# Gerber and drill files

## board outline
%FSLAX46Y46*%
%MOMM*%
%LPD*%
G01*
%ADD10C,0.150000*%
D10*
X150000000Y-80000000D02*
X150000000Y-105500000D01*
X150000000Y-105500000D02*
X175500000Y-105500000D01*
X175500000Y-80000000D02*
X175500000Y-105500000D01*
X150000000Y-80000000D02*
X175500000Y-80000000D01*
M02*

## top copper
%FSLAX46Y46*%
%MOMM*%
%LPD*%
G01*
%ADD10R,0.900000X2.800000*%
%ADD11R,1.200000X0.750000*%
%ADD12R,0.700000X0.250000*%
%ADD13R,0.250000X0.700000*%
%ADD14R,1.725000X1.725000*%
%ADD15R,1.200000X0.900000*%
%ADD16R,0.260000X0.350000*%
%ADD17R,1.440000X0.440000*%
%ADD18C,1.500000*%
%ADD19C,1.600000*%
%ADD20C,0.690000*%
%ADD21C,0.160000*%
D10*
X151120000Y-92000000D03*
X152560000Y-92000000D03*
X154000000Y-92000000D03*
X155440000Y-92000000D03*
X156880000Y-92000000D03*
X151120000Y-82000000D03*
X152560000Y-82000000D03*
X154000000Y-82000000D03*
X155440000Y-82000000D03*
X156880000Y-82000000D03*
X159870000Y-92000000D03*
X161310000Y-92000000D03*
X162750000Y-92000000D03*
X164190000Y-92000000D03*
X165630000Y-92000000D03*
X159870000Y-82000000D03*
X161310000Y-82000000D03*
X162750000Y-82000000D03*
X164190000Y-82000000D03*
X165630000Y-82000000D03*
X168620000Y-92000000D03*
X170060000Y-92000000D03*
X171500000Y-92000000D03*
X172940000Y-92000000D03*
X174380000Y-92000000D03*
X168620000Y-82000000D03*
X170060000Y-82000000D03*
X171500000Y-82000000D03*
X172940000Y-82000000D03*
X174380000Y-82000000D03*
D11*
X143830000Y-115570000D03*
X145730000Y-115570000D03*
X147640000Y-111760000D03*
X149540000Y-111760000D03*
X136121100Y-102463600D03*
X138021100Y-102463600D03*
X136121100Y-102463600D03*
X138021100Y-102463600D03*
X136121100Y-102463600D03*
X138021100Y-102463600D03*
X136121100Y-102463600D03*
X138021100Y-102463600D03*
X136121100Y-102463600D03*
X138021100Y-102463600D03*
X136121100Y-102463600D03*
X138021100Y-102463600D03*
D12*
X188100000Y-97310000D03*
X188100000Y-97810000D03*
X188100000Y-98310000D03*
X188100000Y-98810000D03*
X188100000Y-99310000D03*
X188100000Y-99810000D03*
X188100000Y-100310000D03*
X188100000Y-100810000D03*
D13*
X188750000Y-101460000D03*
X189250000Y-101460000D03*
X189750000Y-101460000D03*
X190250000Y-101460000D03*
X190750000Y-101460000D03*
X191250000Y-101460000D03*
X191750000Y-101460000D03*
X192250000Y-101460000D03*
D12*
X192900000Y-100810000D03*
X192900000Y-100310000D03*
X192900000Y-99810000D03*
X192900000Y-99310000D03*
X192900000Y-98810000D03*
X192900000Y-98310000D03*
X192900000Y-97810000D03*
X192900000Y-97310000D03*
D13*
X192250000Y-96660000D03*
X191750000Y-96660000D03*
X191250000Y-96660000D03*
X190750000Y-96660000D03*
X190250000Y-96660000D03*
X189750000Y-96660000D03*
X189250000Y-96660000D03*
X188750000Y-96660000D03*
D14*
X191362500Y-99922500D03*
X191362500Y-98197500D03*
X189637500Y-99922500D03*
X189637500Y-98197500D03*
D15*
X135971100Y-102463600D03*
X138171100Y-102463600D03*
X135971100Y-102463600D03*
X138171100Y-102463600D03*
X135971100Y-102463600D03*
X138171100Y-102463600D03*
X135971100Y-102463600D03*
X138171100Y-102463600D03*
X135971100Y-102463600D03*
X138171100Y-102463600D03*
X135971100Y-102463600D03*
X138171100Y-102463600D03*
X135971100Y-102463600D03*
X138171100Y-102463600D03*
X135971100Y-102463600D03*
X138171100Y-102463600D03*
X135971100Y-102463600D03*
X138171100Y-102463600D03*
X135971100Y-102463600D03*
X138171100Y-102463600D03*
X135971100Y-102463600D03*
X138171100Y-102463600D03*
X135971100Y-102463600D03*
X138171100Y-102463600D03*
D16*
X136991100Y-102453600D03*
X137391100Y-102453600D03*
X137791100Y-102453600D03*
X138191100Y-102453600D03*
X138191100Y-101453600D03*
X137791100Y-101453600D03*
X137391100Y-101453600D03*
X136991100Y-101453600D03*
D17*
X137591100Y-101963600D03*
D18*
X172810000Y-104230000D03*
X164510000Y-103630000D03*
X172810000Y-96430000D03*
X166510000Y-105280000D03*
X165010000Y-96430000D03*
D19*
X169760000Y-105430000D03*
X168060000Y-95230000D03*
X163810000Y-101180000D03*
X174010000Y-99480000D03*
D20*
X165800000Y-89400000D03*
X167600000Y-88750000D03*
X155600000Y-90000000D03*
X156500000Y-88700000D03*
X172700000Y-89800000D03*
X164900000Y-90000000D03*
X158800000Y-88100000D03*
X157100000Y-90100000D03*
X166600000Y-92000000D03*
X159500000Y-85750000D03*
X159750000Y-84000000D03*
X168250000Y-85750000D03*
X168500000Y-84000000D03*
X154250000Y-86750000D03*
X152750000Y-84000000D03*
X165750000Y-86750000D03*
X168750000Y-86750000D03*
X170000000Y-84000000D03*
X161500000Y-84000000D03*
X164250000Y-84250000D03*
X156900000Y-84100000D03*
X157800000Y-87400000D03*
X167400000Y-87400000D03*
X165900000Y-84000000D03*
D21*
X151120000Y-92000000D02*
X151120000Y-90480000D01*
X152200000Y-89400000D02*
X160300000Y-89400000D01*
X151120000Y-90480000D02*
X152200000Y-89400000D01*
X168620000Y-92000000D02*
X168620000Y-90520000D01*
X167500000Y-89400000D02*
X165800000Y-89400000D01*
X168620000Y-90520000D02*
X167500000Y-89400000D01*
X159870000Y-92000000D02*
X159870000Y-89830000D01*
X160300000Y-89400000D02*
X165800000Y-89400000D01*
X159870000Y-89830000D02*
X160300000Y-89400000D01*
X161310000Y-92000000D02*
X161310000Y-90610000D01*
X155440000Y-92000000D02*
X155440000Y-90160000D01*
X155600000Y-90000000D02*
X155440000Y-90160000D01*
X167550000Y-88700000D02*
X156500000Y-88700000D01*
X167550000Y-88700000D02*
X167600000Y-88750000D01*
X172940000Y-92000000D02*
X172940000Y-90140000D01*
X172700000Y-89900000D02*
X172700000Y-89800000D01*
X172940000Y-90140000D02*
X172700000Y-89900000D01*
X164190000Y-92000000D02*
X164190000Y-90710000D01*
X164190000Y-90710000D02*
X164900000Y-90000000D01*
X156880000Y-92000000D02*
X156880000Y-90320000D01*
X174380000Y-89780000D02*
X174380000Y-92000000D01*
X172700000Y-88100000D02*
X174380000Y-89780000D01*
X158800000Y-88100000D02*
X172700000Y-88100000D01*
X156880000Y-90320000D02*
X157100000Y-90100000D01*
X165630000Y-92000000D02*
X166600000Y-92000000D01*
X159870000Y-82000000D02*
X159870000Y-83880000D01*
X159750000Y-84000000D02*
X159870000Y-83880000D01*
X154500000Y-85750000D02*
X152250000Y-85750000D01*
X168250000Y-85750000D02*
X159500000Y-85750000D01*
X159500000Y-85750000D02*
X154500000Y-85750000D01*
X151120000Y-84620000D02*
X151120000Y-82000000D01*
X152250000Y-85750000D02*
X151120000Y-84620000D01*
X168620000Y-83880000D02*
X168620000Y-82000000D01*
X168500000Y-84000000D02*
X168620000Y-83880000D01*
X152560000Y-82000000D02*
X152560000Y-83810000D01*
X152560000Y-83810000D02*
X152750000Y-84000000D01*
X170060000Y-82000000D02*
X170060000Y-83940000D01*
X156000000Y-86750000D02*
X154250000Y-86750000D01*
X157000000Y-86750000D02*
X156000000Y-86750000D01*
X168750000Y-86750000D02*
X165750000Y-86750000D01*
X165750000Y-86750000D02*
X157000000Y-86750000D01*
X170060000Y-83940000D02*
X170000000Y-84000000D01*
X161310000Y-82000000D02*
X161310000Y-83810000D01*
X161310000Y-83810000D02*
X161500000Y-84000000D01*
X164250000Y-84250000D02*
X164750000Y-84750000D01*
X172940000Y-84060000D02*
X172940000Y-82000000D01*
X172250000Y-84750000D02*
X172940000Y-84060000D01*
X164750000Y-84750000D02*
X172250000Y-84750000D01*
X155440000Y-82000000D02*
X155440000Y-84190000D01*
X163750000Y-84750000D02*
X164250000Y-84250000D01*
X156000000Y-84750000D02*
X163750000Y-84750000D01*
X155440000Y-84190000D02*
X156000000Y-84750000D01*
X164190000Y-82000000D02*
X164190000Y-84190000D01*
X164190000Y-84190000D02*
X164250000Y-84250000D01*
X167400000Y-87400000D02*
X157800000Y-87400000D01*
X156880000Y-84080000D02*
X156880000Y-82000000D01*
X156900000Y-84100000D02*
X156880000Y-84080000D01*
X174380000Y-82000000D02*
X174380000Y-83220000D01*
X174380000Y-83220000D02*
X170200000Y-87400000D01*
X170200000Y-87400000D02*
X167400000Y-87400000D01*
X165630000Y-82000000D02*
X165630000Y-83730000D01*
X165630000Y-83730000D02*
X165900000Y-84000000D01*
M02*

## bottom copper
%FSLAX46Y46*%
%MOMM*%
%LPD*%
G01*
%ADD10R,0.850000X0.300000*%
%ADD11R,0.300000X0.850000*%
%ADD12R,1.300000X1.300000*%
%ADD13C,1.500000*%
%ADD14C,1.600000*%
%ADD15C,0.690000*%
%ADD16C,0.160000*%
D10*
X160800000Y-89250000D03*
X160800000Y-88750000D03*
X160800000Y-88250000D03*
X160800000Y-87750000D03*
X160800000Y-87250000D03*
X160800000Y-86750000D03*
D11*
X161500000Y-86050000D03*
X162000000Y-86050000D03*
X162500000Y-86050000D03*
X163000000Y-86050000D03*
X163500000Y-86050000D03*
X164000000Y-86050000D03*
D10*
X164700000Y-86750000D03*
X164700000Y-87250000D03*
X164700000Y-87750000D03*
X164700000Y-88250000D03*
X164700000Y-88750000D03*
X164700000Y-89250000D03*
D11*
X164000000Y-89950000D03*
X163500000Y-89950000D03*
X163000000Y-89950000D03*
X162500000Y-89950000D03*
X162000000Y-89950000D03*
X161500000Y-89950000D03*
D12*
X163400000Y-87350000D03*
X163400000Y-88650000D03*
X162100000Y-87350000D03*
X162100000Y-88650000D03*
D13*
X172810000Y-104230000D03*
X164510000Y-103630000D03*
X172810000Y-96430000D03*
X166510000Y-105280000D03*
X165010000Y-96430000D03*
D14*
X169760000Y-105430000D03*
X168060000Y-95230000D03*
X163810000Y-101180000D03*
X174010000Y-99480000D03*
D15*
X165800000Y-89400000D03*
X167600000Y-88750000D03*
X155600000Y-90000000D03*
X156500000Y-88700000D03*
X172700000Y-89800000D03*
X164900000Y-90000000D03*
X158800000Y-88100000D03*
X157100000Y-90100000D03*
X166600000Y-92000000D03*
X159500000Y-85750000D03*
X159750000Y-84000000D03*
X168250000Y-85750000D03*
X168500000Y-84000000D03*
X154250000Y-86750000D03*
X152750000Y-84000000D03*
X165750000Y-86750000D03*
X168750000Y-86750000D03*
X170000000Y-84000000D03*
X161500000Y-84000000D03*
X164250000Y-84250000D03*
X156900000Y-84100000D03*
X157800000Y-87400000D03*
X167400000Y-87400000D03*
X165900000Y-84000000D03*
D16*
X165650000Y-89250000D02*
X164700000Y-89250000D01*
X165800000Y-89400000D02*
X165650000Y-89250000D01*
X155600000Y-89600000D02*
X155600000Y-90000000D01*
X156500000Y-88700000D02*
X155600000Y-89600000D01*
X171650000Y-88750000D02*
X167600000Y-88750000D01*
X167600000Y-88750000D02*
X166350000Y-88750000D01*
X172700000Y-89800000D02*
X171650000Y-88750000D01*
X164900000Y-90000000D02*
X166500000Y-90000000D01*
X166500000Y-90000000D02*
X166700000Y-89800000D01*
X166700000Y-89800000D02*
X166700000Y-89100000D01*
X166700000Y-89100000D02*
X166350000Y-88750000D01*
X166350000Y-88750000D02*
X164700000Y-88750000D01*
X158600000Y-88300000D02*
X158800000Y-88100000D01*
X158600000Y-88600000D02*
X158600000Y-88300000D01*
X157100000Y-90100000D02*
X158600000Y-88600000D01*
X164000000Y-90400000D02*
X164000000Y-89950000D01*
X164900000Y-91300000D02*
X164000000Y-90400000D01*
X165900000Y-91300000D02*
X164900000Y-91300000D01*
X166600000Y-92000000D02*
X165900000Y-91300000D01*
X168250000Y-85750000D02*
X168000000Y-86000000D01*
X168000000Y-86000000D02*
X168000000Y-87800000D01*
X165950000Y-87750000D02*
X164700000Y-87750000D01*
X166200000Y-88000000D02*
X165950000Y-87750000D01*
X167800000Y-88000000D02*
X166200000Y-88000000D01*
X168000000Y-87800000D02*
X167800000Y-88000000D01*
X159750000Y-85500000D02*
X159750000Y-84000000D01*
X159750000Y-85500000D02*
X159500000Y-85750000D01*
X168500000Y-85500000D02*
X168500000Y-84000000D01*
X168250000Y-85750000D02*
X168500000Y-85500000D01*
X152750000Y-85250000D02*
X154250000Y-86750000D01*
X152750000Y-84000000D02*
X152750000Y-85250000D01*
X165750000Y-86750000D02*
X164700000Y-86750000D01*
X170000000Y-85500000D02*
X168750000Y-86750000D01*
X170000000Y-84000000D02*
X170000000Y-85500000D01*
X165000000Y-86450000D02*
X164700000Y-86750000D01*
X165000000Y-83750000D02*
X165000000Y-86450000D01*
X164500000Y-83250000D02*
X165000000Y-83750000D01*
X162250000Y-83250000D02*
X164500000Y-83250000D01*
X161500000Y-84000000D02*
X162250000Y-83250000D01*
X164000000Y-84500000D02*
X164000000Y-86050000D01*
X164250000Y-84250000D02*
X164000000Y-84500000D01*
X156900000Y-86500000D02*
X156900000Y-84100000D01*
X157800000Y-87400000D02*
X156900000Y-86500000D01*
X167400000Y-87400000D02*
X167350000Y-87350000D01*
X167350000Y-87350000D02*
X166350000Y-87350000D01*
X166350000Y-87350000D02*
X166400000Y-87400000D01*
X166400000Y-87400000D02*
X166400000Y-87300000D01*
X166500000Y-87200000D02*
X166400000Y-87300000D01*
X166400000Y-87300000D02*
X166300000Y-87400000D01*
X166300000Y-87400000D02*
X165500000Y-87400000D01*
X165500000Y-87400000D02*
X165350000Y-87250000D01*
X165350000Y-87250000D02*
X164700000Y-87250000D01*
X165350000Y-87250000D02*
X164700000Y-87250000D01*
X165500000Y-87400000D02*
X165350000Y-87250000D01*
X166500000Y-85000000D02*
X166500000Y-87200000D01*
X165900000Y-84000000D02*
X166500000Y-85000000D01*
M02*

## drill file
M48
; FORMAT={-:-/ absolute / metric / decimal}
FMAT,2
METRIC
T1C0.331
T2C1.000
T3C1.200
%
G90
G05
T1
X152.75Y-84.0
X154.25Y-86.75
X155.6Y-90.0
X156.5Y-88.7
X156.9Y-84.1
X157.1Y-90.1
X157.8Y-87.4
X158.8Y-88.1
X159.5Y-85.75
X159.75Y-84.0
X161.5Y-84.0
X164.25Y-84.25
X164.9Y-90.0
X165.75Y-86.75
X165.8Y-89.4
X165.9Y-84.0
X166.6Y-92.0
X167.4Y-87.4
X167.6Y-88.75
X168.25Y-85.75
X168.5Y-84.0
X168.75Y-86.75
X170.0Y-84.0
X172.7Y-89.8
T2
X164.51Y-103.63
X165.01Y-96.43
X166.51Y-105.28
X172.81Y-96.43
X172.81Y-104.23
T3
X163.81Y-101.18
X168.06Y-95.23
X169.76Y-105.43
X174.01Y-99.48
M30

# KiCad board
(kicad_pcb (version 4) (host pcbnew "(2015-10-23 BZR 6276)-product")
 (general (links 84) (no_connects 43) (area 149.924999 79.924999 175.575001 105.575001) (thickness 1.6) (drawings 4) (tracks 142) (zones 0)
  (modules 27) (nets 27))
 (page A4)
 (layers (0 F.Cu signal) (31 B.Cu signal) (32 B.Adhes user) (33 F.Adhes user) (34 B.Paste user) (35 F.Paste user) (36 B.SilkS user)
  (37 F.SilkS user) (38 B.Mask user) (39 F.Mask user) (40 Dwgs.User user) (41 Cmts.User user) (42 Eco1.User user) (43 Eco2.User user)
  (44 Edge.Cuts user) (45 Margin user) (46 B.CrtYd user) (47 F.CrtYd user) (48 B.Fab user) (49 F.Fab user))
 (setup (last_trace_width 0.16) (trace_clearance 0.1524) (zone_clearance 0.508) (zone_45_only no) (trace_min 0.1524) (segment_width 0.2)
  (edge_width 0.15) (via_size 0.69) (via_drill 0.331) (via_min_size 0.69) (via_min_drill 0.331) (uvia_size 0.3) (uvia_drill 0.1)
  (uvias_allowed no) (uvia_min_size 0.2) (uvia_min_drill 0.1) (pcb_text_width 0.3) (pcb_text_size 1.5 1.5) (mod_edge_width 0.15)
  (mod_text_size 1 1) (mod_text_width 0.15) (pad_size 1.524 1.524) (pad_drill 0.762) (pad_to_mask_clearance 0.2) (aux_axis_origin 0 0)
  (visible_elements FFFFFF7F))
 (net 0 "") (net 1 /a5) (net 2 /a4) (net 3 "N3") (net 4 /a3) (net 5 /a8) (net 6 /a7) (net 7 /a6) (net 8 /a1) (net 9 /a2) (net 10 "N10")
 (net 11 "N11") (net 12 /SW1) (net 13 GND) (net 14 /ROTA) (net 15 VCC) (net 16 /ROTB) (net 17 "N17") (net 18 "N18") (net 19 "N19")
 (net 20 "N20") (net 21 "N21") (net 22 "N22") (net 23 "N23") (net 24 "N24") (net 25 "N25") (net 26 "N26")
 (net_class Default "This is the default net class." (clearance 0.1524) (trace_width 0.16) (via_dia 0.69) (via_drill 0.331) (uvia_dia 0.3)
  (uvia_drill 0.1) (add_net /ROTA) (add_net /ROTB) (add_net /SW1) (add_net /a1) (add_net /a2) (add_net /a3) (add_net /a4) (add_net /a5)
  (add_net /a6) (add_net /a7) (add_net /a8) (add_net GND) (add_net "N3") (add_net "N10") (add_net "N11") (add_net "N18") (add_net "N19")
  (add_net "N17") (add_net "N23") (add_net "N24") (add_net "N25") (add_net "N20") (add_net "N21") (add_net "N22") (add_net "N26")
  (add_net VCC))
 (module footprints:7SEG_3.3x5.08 (layer F.Cu) (at 154 87 90)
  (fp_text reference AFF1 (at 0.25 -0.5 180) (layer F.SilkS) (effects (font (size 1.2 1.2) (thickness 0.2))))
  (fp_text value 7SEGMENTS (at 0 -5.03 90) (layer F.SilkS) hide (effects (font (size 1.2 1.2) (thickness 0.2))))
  (pad 1 smd rect (at -5 -2.88 90) (size 2.8 0.9) (layers F.Cu F.Paste F.Mask) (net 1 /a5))
  (pad 2 smd rect (at -5 -1.44 90) (size 2.8 0.9) (layers F.Cu F.Paste F.Mask) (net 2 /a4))
  (pad 3 smd rect (at -5 0 90) (size 2.8 0.9) (layers F.Cu F.Paste F.Mask) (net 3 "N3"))
  (pad 4 smd rect (at -5 1.44 90) (size 2.8 0.9) (layers F.Cu F.Paste F.Mask) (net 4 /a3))
  (pad 5 smd rect (at -5 2.88 90) (size 2.8 0.9) (layers F.Cu F.Paste F.Mask) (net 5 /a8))
  (pad 10 smd rect (at 5 -2.88 90) (size 2.8 0.9) (layers F.Cu F.Paste F.Mask) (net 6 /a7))
  (pad 9 smd rect (at 5 -1.44 90) (size 2.8 0.9) (layers F.Cu F.Paste F.Mask) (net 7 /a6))
  (pad 8 smd rect (at 5 0 90) (size 2.8 0.9) (layers F.Cu F.Paste F.Mask) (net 3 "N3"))
  (pad 7 smd rect (at 5 1.44 90) (size 2.8 0.9) (layers F.Cu F.Paste F.Mask) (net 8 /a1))
  (pad 6 smd rect (at 5 2.88 90) (size 2.8 0.9) (layers F.Cu F.Paste F.Mask) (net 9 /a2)))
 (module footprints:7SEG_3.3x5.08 (layer F.Cu) (at 162.75 87 90)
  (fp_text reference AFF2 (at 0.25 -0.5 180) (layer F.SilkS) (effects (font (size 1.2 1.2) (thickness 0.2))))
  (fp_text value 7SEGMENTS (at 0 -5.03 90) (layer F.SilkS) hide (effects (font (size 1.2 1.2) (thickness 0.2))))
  (pad 1 smd rect (at -5 -2.88 90) (size 2.8 0.9) (layers F.Cu F.Paste F.Mask) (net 1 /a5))
  (pad 2 smd rect (at -5 -1.44 90) (size 2.8 0.9) (layers F.Cu F.Paste F.Mask) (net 2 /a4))
  (pad 3 smd rect (at -5 0 90) (size 2.8 0.9) (layers F.Cu F.Paste F.Mask) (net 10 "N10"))
  (pad 4 smd rect (at -5 1.44 90) (size 2.8 0.9) (layers F.Cu F.Paste F.Mask) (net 4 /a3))
  (pad 5 smd rect (at -5 2.88 90) (size 2.8 0.9) (layers F.Cu F.Paste F.Mask) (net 5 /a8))
  (pad 10 smd rect (at 5 -2.88 90) (size 2.8 0.9) (layers F.Cu F.Paste F.Mask) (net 6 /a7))
  (pad 9 smd rect (at 5 -1.44 90) (size 2.8 0.9) (layers F.Cu F.Paste F.Mask) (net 7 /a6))
  (pad 8 smd rect (at 5 0 90) (size 2.8 0.9) (layers F.Cu F.Paste F.Mask) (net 10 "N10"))
  (pad 7 smd rect (at 5 1.44 90) (size 2.8 0.9) (layers F.Cu F.Paste F.Mask) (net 8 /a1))
  (pad 6 smd rect (at 5 2.88 90) (size 2.8 0.9) (layers F.Cu F.Paste F.Mask) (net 9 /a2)))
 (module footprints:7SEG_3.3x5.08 (layer F.Cu) (at 171.5 87 90)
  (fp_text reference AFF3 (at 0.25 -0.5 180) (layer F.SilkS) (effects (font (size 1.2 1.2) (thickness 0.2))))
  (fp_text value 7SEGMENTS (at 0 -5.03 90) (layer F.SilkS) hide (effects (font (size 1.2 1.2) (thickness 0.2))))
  (pad 1 smd rect (at -5 -2.88 90) (size 2.8 0.9) (layers F.Cu F.Paste F.Mask) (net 1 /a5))
  (pad 2 smd rect (at -5 -1.44 90) (size 2.8 0.9) (layers F.Cu F.Paste F.Mask) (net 2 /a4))
  (pad 3 smd rect (at -5 0 90) (size 2.8 0.9) (layers F.Cu F.Paste F.Mask) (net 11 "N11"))
  (pad 4 smd rect (at -5 1.44 90) (size 2.8 0.9) (layers F.Cu F.Paste F.Mask) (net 4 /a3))
  (pad 5 smd rect (at -5 2.88 90) (size 2.8 0.9) (layers F.Cu F.Paste F.Mask) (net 5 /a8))
  (pad 10 smd rect (at 5 -2.88 90) (size 2.8 0.9) (layers F.Cu F.Paste F.Mask) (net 6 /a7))
  (pad 9 smd rect (at 5 -1.44 90) (size 2.8 0.9) (layers F.Cu F.Paste F.Mask) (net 7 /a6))
  (pad 8 smd rect (at 5 0 90) (size 2.8 0.9) (layers F.Cu F.Paste F.Mask) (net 11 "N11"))
  (pad 7 smd rect (at 5 1.44 90) (size 2.8 0.9) (layers F.Cu F.Paste F.Mask) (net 8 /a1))
  (pad 6 smd rect (at 5 2.88 90) (size 2.8 0.9) (layers F.Cu F.Paste F.Mask) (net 9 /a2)))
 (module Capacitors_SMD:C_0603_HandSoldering (layer F.Cu) (at 144.78 115.57)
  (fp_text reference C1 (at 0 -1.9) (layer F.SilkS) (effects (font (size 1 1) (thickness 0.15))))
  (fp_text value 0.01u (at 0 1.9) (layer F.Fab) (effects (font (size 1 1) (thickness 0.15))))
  (pad 1 smd rect (at -0.95 0) (size 1.2 0.75) (layers F.Cu F.Paste F.Mask) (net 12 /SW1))
  (pad 2 smd rect (at 0.95 0) (size 1.2 0.75) (layers F.Cu F.Paste F.Mask) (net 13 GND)))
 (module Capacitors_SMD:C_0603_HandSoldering (layer F.Cu) (at 148.59 111.76)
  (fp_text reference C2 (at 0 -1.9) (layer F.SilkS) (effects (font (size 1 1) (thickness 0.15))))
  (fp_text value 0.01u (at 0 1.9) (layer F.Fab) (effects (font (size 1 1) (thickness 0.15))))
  (pad 1 smd rect (at -0.95 0) (size 1.2 0.75) (layers F.Cu F.Paste F.Mask) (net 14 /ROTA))
  (pad 2 smd rect (at 0.95 0) (size 1.2 0.75) (layers F.Cu F.Paste F.Mask) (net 13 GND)))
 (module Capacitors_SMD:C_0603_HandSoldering (layer F.Cu) (at 137.0711 102.4636)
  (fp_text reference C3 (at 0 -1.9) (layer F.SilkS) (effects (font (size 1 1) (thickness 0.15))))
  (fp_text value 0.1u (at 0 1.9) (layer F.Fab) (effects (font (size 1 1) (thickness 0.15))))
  (pad 1 smd rect (at -0.95 0) (size 1.2 0.75) (layers F.Cu F.Paste F.Mask) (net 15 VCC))
  (pad 2 smd rect (at 0.95 0) (size 1.2 0.75) (layers F.Cu F.Paste F.Mask) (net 13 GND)))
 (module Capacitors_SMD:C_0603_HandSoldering (layer F.Cu) (at 137.0711 102.4636)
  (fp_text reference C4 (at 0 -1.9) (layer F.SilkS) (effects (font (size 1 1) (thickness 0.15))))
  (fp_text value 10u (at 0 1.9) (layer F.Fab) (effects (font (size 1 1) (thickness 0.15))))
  (pad 1 smd rect (at -0.95 0) (size 1.2 0.75) (layers F.Cu F.Paste F.Mask) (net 15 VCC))
  (pad 2 smd rect (at 0.95 0) (size 1.2 0.75) (layers F.Cu F.Paste F.Mask) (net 13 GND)))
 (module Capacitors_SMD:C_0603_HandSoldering (layer F.Cu) (at 137.0711 102.4636)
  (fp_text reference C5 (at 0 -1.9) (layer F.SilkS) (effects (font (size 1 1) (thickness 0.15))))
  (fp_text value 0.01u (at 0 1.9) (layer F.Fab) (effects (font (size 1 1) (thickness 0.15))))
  (pad 1 smd rect (at -0.95 0) (size 1.2 0.75) (layers F.Cu F.Paste F.Mask) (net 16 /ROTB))
  (pad 2 smd rect (at 0.95 0) (size 1.2 0.75) (layers F.Cu F.Paste F.Mask) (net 13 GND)))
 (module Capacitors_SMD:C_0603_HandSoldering (layer F.Cu) (at 137.0711 102.4636)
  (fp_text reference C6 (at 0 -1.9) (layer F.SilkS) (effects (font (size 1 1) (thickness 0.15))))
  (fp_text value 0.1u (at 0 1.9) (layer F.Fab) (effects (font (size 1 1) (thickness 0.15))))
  (pad 1 smd rect (at -0.95 0) (size 1.2 0.75) (layers F.Cu F.Paste F.Mask) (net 13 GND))
  (pad 2 smd rect (at 0.95 0) (size 1.2 0.75) (layers F.Cu F.Paste F.Mask) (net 15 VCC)))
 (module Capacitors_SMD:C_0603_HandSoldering (layer F.Cu) (at 137.0711 102.4636)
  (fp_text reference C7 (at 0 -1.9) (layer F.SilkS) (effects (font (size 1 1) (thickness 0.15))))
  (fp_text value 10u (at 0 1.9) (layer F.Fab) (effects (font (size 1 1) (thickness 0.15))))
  (pad 1 smd rect (at -0.95 0) (size 1.2 0.75) (layers F.Cu F.Paste F.Mask) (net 13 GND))
  (pad 2 smd rect (at 0.95 0) (size 1.2 0.75) (layers F.Cu F.Paste F.Mask) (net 15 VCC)))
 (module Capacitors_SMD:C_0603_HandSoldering (layer F.Cu) (at 137.0711 102.4636)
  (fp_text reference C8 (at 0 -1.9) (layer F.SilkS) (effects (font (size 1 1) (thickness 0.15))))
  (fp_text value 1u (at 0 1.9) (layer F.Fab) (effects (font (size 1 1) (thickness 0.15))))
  (pad 1 smd rect (at -0.95 0) (size 1.2 0.75) (layers F.Cu F.Paste F.Mask) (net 15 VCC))
  (pad 2 smd rect (at 0.95 0) (size 1.2 0.75) (layers F.Cu F.Paste F.Mask) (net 13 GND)))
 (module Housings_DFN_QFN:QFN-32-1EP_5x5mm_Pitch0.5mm (layer F.Cu) (at 190.5 99.06)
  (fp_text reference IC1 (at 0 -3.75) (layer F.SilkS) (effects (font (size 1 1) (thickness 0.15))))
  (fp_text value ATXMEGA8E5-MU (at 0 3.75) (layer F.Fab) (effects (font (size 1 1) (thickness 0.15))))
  (pad 1 smd rect (at -2.4 -1.75) (size 0.7 0.25) (layers F.Cu F.Paste F.Mask) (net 13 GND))
  (pad 2 smd rect (at -2.4 -1.25) (size 0.7 0.25) (layers F.Cu F.Paste F.Mask))
  (pad 3 smd rect (at -2.4 -0.75) (size 0.7 0.25) (layers F.Cu F.Paste F.Mask))
  (pad 4 smd rect (at -2.4 -0.25) (size 0.7 0.25) (layers F.Cu F.Paste F.Mask))
  (pad 5 smd rect (at -2.4 0.25) (size 0.7 0.25) (layers F.Cu F.Paste F.Mask))
  (pad 6 smd rect (at -2.4 0.75) (size 0.7 0.25) (layers F.Cu F.Paste F.Mask))
  (pad 7 smd rect (at -2.4 1.25) (size 0.7 0.25) (layers F.Cu F.Paste F.Mask))
  (pad 8 smd rect (at -2.4 1.75) (size 0.7 0.25) (layers F.Cu F.Paste F.Mask) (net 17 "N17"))
  (pad 9 smd rect (at -1.75 2.4 90) (size 0.7 0.25) (layers F.Cu F.Paste F.Mask))
  (pad 10 smd rect (at -1.25 2.4 90) (size 0.7 0.25) (layers F.Cu F.Paste F.Mask))
  (pad 11 smd rect (at -0.75 2.4 90) (size 0.7 0.25) (layers F.Cu F.Paste F.Mask))
  (pad 12 smd rect (at -0.25 2.4 90) (size 0.7 0.25) (layers F.Cu F.Paste F.Mask))
  (pad 13 smd rect (at 0.25 2.4 90) (size 0.7 0.25) (layers F.Cu F.Paste F.Mask))
  (pad 14 smd rect (at 0.75 2.4 90) (size 0.7 0.25) (layers F.Cu F.Paste F.Mask))
  (pad 15 smd rect (at 1.25 2.4 90) (size 0.7 0.25) (layers F.Cu F.Paste F.Mask) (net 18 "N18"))
  (pad 16 smd rect (at 1.75 2.4 90) (size 0.7 0.25) (layers F.Cu F.Paste F.Mask) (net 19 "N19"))
  (pad 17 smd rect (at 2.4 1.75) (size 0.7 0.25) (layers F.Cu F.Paste F.Mask) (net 15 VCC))
  (pad 18 smd rect (at 2.4 1.25) (size 0.7 0.25) (layers F.Cu F.Paste F.Mask) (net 13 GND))
  (pad 19 smd rect (at 2.4 0.75) (size 0.7 0.25) (layers F.Cu F.Paste F.Mask))
  (pad 20 smd rect (at 2.4 0.25) (size 0.7 0.25) (layers F.Cu F.Paste F.Mask))
  (pad 21 smd rect (at 2.4 -0.25) (size 0.7 0.25) (layers F.Cu F.Paste F.Mask))
  (pad 22 smd rect (at 2.4 -0.75) (size 0.7 0.25) (layers F.Cu F.Paste F.Mask))
  (pad 23 smd rect (at 2.4 -1.25) (size 0.7 0.25) (layers F.Cu F.Paste F.Mask))
  (pad 24 smd rect (at 2.4 -1.75) (size 0.7 0.25) (layers F.Cu F.Paste F.Mask))
  (pad 25 smd rect (at 1.75 -2.4 90) (size 0.7 0.25) (layers F.Cu F.Paste F.Mask))
  (pad 26 smd rect (at 1.25 -2.4 90) (size 0.7 0.25) (layers F.Cu F.Paste F.Mask) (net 12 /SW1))
  (pad 27 smd rect (at 0.75 -2.4 90) (size 0.7 0.25) (layers F.Cu F.Paste F.Mask) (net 16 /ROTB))
  (pad 28 smd rect (at 0.25 -2.4 90) (size 0.7 0.25) (layers F.Cu F.Paste F.Mask) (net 14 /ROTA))
  (pad 29 smd rect (at -0.25 -2.4 90) (size 0.7 0.25) (layers F.Cu F.Paste F.Mask))
  (pad 30 smd rect (at -0.75 -2.4 90) (size 0.7 0.25) (layers F.Cu F.Paste F.Mask))
  (pad 31 smd rect (at -1.25 -2.4 90) (size 0.7 0.25) (layers F.Cu F.Paste F.Mask))
  (pad 32 smd rect (at -1.75 -2.4 90) (size 0.7 0.25) (layers F.Cu F.Paste F.Mask) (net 15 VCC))
  (pad 33 smd rect (at 0.8625 0.8625) (size 1.725 1.725) (layers F.Cu F.Paste F.Mask) (solder_paste_margin_ratio -0.2))
  (pad 33 smd rect (at 0.8625 -0.8625) (size 1.725 1.725) (layers F.Cu F.Paste F.Mask) (solder_paste_margin_ratio -0.2))
  (pad 33 smd rect (at -0.8625 0.8625) (size 1.725 1.725) (layers F.Cu F.Paste F.Mask) (solder_paste_margin_ratio -0.2))
  (pad 33 smd rect (at -0.8625 -0.8625) (size 1.725 1.725) (layers F.Cu F.Paste F.Mask) (solder_paste_margin_ratio -0.2)))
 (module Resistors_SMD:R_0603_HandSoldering (layer F.Cu) (at 137.0711 102.4636)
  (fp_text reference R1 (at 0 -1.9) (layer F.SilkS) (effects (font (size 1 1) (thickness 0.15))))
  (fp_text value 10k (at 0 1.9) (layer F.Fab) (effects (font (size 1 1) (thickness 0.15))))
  (pad 1 smd rect (at -1.1 0) (size 1.2 0.9) (layers F.Cu F.Paste F.Mask) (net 15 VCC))
  (pad 2 smd rect (at 1.1 0) (size 1.2 0.9) (layers F.Cu F.Paste F.Mask) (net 17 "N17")))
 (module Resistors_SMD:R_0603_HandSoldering (layer F.Cu) (at 137.0711 102.4636)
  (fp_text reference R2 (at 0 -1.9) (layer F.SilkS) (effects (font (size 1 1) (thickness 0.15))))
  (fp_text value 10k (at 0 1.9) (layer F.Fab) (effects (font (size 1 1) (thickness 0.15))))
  (pad 1 smd rect (at -1.1 0) (size 1.2 0.9) (layers F.Cu F.Paste F.Mask) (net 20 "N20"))
  (pad 2 smd rect (at 1.1 0) (size 1.2 0.9) (layers F.Cu F.Paste F.Mask) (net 12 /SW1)))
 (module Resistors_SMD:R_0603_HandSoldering (layer F.Cu) (at 137.0711 102.4636)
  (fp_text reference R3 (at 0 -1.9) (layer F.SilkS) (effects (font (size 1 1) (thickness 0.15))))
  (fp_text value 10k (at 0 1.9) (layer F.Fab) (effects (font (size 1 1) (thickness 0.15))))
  (pad 1 smd rect (at -1.1 0) (size 1.2 0.9) (layers F.Cu F.Paste F.Mask) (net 20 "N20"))
  (pad 2 smd rect (at 1.1 0) (size 1.2 0.9) (layers F.Cu F.Paste F.Mask) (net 15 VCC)))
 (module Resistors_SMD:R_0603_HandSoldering (layer F.Cu) (at 137.0711 102.4636)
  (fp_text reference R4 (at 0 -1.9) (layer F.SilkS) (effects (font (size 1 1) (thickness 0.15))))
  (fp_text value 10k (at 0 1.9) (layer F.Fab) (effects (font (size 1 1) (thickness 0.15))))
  (pad 1 smd rect (at -1.1 0) (size 1.2 0.9) (layers F.Cu F.Paste F.Mask) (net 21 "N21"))
  (pad 2 smd rect (at 1.1 0) (size 1.2 0.9) (layers F.Cu F.Paste F.Mask) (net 14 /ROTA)))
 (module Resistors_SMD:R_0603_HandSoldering (layer F.Cu) (at 137.0711 102.4636)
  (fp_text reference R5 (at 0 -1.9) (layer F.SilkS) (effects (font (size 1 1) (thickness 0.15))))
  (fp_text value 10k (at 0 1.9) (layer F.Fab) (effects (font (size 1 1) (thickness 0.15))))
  (pad 1 smd rect (at -1.1 0) (size 1.2 0.9) (layers F.Cu F.Paste F.Mask) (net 21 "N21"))
  (pad 2 smd rect (at 1.1 0) (size 1.2 0.9) (layers F.Cu F.Paste F.Mask) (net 15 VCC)))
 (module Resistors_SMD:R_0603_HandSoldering (layer F.Cu) (at 137.0711 102.4636)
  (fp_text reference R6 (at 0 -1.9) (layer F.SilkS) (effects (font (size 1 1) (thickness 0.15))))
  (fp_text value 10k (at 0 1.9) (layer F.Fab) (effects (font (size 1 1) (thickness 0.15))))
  (pad 1 smd rect (at -1.1 0) (size 1.2 0.9) (layers F.Cu F.Paste F.Mask) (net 15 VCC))
  (pad 2 smd rect (at 1.1 0) (size 1.2 0.9) (layers F.Cu F.Paste F.Mask) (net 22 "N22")))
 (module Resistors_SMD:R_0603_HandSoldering (layer F.Cu) (at 137.0711 102.4636)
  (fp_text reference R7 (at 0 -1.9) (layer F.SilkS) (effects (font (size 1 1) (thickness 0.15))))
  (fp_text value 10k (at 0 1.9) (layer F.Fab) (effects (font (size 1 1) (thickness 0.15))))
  (pad 1 smd rect (at -1.1 0) (size 1.2 0.9) (layers F.Cu F.Paste F.Mask) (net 16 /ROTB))
  (pad 2 smd rect (at 1.1 0) (size 1.2 0.9) (layers F.Cu F.Paste F.Mask) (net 22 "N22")))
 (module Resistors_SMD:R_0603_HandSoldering (layer F.Cu) (at 137.0711 102.4636)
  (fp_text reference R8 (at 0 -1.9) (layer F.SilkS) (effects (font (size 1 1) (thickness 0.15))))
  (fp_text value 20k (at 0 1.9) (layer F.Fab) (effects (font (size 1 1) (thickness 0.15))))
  (pad 1 smd rect (at -1.1 0) (size 1.2 0.9) (layers F.Cu F.Paste F.Mask) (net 15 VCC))
  (pad 2 smd rect (at 1.1 0) (size 1.2 0.9) (layers F.Cu F.Paste F.Mask) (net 18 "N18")))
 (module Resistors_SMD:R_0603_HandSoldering (layer F.Cu) (at 137.0711 102.4636)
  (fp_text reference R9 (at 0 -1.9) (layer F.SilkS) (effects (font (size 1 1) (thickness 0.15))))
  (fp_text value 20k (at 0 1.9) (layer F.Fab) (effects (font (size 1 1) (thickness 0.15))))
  (pad 1 smd rect (at -1.1 0) (size 1.2 0.9) (layers F.Cu F.Paste F.Mask) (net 15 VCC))
  (pad 2 smd rect (at 1.1 0) (size 1.2 0.9) (layers F.Cu F.Paste F.Mask) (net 19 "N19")))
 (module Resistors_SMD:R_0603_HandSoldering (layer F.Cu) (at 137.0711 102.4636)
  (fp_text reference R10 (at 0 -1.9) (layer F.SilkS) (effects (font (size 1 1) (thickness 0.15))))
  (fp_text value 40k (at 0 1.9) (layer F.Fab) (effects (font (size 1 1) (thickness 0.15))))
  (pad 1 smd rect (at -1.1 0) (size 1.2 0.9) (layers F.Cu F.Paste F.Mask) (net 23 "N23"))
  (pad 2 smd rect (at 1.1 0) (size 1.2 0.9) (layers F.Cu F.Paste F.Mask) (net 15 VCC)))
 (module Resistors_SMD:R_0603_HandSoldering (layer F.Cu) (at 137.0711 102.4636)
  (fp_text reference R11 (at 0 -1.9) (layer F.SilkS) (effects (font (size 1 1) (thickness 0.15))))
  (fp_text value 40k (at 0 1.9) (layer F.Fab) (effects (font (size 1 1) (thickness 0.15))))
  (pad 1 smd rect (at -1.1 0) (size 1.2 0.9) (layers F.Cu F.Paste F.Mask) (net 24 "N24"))
  (pad 2 smd rect (at 1.1 0) (size 1.2 0.9) (layers F.Cu F.Paste F.Mask) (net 15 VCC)))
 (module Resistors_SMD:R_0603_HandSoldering (layer F.Cu) (at 137.0711 102.4636)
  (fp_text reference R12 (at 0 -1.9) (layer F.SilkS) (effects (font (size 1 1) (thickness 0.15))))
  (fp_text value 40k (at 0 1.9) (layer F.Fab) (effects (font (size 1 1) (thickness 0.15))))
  (pad 1 smd rect (at -1.1 0) (size 1.2 0.9) (layers F.Cu F.Paste F.Mask) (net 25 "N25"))
  (pad 2 smd rect (at 1.1 0) (size 1.2 0.9) (layers F.Cu F.Paste F.Mask) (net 15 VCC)))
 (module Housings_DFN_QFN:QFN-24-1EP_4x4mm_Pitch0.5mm (layer B.Cu) (at 162.75 88)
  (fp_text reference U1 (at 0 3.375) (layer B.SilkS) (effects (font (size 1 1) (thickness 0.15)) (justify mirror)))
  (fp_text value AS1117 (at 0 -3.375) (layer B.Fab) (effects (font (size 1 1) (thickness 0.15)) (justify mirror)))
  (pad 1 smd rect (at -1.95 1.25) (size 0.85 0.3) (layers B.Cu B.Paste B.Mask) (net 11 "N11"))
  (pad 2 smd rect (at -1.95 0.75) (size 0.85 0.3) (layers B.Cu B.Paste B.Mask))
  (pad 3 smd rect (at -1.95 0.25) (size 0.85 0.3) (layers B.Cu B.Paste B.Mask) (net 13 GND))
  (pad 4 smd rect (at -1.95 -0.25) (size 0.85 0.3) (layers B.Cu B.Paste B.Mask))
  (pad 5 smd rect (at -1.95 -0.75) (size 0.85 0.3) (layers B.Cu B.Paste B.Mask))
  (pad 6 smd rect (at -1.95 -1.25) (size 0.85 0.3) (layers B.Cu B.Paste B.Mask))
  (pad 7 smd rect (at -1.25 -1.95 270) (size 0.85 0.3) (layers B.Cu B.Paste B.Mask))
  (pad 8 smd rect (at -0.75 -1.95 270) (size 0.85 0.3) (layers B.Cu B.Paste B.Mask))
  (pad 9 smd rect (at -0.25 -1.95 270) (size 0.85 0.3) (layers B.Cu B.Paste B.Mask) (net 24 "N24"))
  (pad 10 smd rect (at 0.25 -1.95 270) (size 0.85 0.3) (layers B.Cu B.Paste B.Mask) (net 25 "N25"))
  (pad 11 smd rect (at 0.75 -1.95 270) (size 0.85 0.3) (layers B.Cu B.Paste B.Mask) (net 18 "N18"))
  (pad 12 smd rect (at 1.25 -1.95 270) (size 0.85 0.3) (layers B.Cu B.Paste B.Mask) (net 8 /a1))
  (pad 13 smd rect (at 1.95 -1.25) (size 0.85 0.3) (layers B.Cu B.Paste B.Mask) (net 7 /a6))
  (pad 14 smd rect (at 1.95 -0.75) (size 0.85 0.3) (layers B.Cu B.Paste B.Mask) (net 9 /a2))
  (pad 15 smd rect (at 1.95 -0.25) (size 0.85 0.3) (layers B.Cu B.Paste B.Mask) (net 6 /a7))
  (pad 16 smd rect (at 1.95 0.25) (size 0.85 0.3) (layers B.Cu B.Paste B.Mask) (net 15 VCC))
  (pad 17 smd rect (at 1.95 0.75) (size 0.85 0.3) (layers B.Cu B.Paste B.Mask) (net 4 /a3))
  (pad 18 smd rect (at 1.95 1.25) (size 0.85 0.3) (layers B.Cu B.Paste B.Mask) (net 1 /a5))
  (pad 19 smd rect (at 1.25 1.95 270) (size 0.85 0.3) (layers B.Cu B.Paste B.Mask) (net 5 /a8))
  (pad 20 smd rect (at 0.75 1.95 270) (size 0.85 0.3) (layers B.Cu B.Paste B.Mask) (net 2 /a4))
  (pad 21 smd rect (at 0.25 1.95 270) (size 0.85 0.3) (layers B.Cu B.Paste B.Mask) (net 23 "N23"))
  (pad 22 smd rect (at -0.25 1.95 270) (size 0.85 0.3) (layers B.Cu B.Paste B.Mask) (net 19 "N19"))
  (pad 23 smd rect (at -0.75 1.95 270) (size 0.85 0.3) (layers B.Cu B.Paste B.Mask) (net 3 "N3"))
  (pad 24 smd rect (at -1.25 1.95 270) (size 0.85 0.3) (layers B.Cu B.Paste B.Mask) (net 10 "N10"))
  (pad 25 smd rect (at 0.65 -0.65) (size 1.3 1.3) (layers B.Cu B.Paste B.Mask) (solder_paste_margin_ratio -0.2))
  (pad 25 smd rect (at 0.65 0.65) (size 1.3 1.3) (layers B.Cu B.Paste B.Mask) (solder_paste_margin_ratio -0.2))
  (pad 25 smd rect (at -0.65 -0.65) (size 1.3 1.3) (layers B.Cu B.Paste B.Mask) (solder_paste_margin_ratio -0.2))
  (pad 25 smd rect (at -0.65 0.65) (size 1.3 1.3) (layers B.Cu B.Paste B.Mask) (solder_paste_margin_ratio -0.2)))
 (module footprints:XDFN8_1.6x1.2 (layer F.Cu) (at 137.0711 102.4636) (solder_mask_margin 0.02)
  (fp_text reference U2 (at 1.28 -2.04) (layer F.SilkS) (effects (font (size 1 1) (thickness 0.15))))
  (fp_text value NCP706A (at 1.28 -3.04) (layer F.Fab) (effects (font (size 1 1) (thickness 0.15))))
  (pad 1 smd rect (at -0.08 -0.01) (size 0.26 0.35) (layers F.Cu F.Paste F.Mask) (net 15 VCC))
  (pad 2 smd rect (at 0.32 -0.01) (size 0.26 0.35) (layers F.Cu F.Paste F.Mask) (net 15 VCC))
  (pad 3 smd rect (at 0.72 -0.01) (size 0.26 0.35) (layers F.Cu F.Paste F.Mask))
  (pad 4 smd rect (at 1.12 -0.01) (size 0.26 0.35) (layers F.Cu F.Paste F.Mask) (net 15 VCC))
  (pad 5 smd rect (at 1.12 -1.01) (size 0.26 0.35) (layers F.Cu F.Paste F.Mask) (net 13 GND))
  (pad 6 smd rect (at 0.72 -1.01) (size 0.26 0.35) (layers F.Cu F.Paste F.Mask) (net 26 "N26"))
  (pad 7 smd rect (at 0.32 -1.01) (size 0.26 0.35) (layers F.Cu F.Paste F.Mask) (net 26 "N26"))
  (pad 8 smd rect (at -0.08 -1.01) (size 0.26 0.35) (layers F.Cu F.Paste F.Mask) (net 26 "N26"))
  (pad 9 smd rect (at 0.52 -0.5) (size 1.44 0.44) (layers F.Cu F.Paste F.Mask)))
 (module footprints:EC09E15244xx (layer F.Cu) (at 168.91 100.33)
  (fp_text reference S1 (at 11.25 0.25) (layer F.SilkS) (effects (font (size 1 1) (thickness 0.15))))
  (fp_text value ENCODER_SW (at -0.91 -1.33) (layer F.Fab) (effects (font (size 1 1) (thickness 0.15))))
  (pad 1 thru_hole circle (at 3.9 3.9) (size 1.5 1.5) (drill 1) (layers *.Cu *.Mask F.SilkS) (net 13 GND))
  (pad 2 thru_hole circle (at -4.4 3.3) (size 1.5 1.5) (drill 1) (layers *.Cu *.Mask F.SilkS) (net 21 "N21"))
  (pad 3 thru_hole circle (at 3.9 -3.9) (size 1.5 1.5) (drill 1) (layers *.Cu *.Mask F.SilkS) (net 22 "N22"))
  (pad 4 thru_hole circle (at -2.4 4.95) (size 1.5 1.5) (drill 1) (layers *.Cu *.Mask F.SilkS) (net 13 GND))
  (pad 5 thru_hole circle (at -3.9 -3.9) (size 1.5 1.5) (drill 1) (layers *.Cu *.Mask F.SilkS) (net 20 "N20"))
  (pad "" np_thru_hole circle (at 0.85 5.1) (size 1.6 1.6) (drill 1.2) (layers *.Cu *.Mask F.SilkS))
  (pad "" np_thru_hole circle (at -0.85 -5.1) (size 1.6 1.6) (drill 1.2) (layers *.Cu *.Mask F.SilkS))
  (pad "" np_thru_hole circle (at -5.1 0.85) (size 1.6 1.6) (drill 1.2) (layers *.Cu *.Mask F.SilkS))
  (pad "" np_thru_hole circle (at 5.1 -0.85) (size 1.6 1.6) (drill 1.2) (layers *.Cu *.Mask F.SilkS)))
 (gr_line (start 150 80) (end 150 105.5) (angle 90) (layer Edge.Cuts) (width 0.15))
 (gr_line (start 150 105.5) (end 175.5 105.5) (angle 90) (layer Edge.Cuts) (width 0.15))
 (gr_line (start 175.5 80) (end 175.5 105.5) (angle 90) (layer Edge.Cuts) (width 0.15))
 (gr_line (start 150 80) (end 175.5 80) (angle 90) (layer Edge.Cuts) (width 0.15))
 (segment (start 151.12 92) (end 151.12 90.48) (width 0.16) (layer F.Cu) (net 1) (status 400000))
 (segment (start 152.2 89.4) (end 160.3 89.4) (width 0.16) (layer F.Cu) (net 1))
 (segment (start 151.12 90.48) (end 152.2 89.4) (width 0.16) (layer F.Cu) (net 1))
 (segment (start 168.62 92) (end 168.62 90.52) (width 0.16) (layer F.Cu) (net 1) (status 400000))
 (segment (start 167.5 89.4) (end 165.8 89.4) (width 0.16) (layer F.Cu) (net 1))
 (segment (start 168.62 90.52) (end 167.5 89.4) (width 0.16) (layer F.Cu) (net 1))
 (segment (start 159.87 92) (end 159.87 89.83) (width 0.16) (layer F.Cu) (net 1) (status 400000))
 (segment (start 165.65 89.25) (end 164.7 89.25) (width 0.16) (layer B.Cu) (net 1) (status 800000))
 (segment (start 165.8 89.4) (end 165.65 89.25) (width 0.16) (layer B.Cu) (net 1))
 (via (at 165.8 89.4) (size 0.69) (drill 0.331) (layers F.Cu B.Cu) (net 1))
 (segment (start 160.3 89.4) (end 165.8 89.4) (width 0.16) (layer F.Cu) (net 1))
 (segment (start 159.87 89.83) (end 160.3 89.4) (width 0.16) (layer F.Cu) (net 1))
 (segment (start 161.31 92) (end 161.31 90.61) (width 0.16) (layer F.Cu) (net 2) (status C00000))
 (via (at 167.6 88.75) (size 0.69) (drill 0.331) (layers F.Cu B.Cu) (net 4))
 (segment (start 155.44 92) (end 155.44 90.16) (width 0.16) (layer F.Cu) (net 4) (status 400000))
 (segment (start 155.6 90) (end 155.44 90.16) (width 0.16) (layer F.Cu) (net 4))
 (via (at 155.6 90) (size 0.69) (drill 0.331) (layers F.Cu B.Cu) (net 4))
 (segment (start 155.6 89.6) (end 155.6 90) (width 0.16) (layer B.Cu) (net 4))
 (segment (start 156.5 88.7) (end 155.6 89.6) (width 0.16) (layer B.Cu) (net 4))
 (via (at 156.5 88.7) (size 0.69) (drill 0.331) (layers F.Cu B.Cu) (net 4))
 (segment (start 167.55 88.7) (end 156.5 88.7) (width 0.16) (layer F.Cu) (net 4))
 (segment (start 167.55 88.7) (end 167.6 88.75) (width 0.16) (layer F.Cu) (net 4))
 (segment (start 172.94 92) (end 172.94 90.14) (width 0.16) (layer F.Cu) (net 4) (status 400000))
 (segment (start 171.65 88.75) (end 167.6 88.75) (width 0.16) (layer B.Cu) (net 4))
 (segment (start 167.6 88.75) (end 166.35 88.75) (width 0.16) (layer B.Cu) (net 4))
 (segment (start 172.7 89.8) (end 171.65 88.75) (width 0.16) (layer B.Cu) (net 4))
 (via (at 172.7 89.8) (size 0.69) (drill 0.331) (layers F.Cu B.Cu) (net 4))
 (segment (start 172.7 89.9) (end 172.7 89.8) (width 0.16) (layer F.Cu) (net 4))
 (segment (start 172.94 90.14) (end 172.7 89.9) (width 0.16) (layer F.Cu) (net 4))
 (segment (start 164.19 92) (end 164.19 90.71) (width 0.16) (layer F.Cu) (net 4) (status C00000))
 (segment (start 164.19 90.71) (end 164.9 90) (width 0.16) (layer F.Cu) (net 4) (status 400000))
 (via (at 164.9 90) (size 0.69) (drill 0.331) (layers F.Cu B.Cu) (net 4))
 (segment (start 164.9 90) (end 166.5 90) (width 0.16) (layer B.Cu) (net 4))
 (segment (start 166.5 90) (end 166.7 89.8) (width 0.16) (layer B.Cu) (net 4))
 (segment (start 166.7 89.8) (end 166.7 89.1) (width 0.16) (layer B.Cu) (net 4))
 (segment (start 166.7 89.1) (end 166.35 88.75) (width 0.16) (layer B.Cu) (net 4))
 (segment (start 166.35 88.75) (end 164.7 88.75) (width 0.16) (layer B.Cu) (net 4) (status 800000))
 (segment (start 156.88 92) (end 156.88 90.32) (width 0.16) (layer F.Cu) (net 5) (status 400000))
 (segment (start 174.38 89.78) (end 174.38 92) (width 0.16) (layer F.Cu) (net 5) (status 800000))
 (segment (start 172.7 88.1) (end 174.38 89.78) (width 0.16) (layer F.Cu) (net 5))
 (segment (start 158.8 88.1) (end 172.7 88.1) (width 0.16) (layer F.Cu) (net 5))
 (via (at 158.8 88.1) (size 0.69) (drill 0.331) (layers F.Cu B.Cu) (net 5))
 (segment (start 158.6 88.3) (end 158.8 88.1) (width 0.16) (layer B.Cu) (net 5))
 (segment (start 158.6 88.6) (end 158.6 88.3) (width 0.16) (layer B.Cu) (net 5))
 (segment (start 157.1 90.1) (end 158.6 88.6) (width 0.16) (layer B.Cu) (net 5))
 (via (at 157.1 90.1) (size 0.69) (drill 0.331) (layers F.Cu B.Cu) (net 5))
 (segment (start 156.88 90.32) (end 157.1 90.1) (width 0.16) (layer F.Cu) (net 5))
 (segment (start 165.63 92) (end 166.6 92) (width 0.16) (layer F.Cu) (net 5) (status 400000))
 (segment (start 164 90.4) (end 164 89.95) (width 0.16) (layer B.Cu) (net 5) (status 800000))
 (segment (start 164.9 91.3) (end 164 90.4) (width 0.16) (layer B.Cu) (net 5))
 (segment (start 165.9 91.3) (end 164.9 91.3) (width 0.16) (layer B.Cu) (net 5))
 (segment (start 166.6 92) (end 165.9 91.3) (width 0.16) (layer B.Cu) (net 5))
 (via (at 166.6 92) (size 0.69) (drill 0.331) (layers F.Cu B.Cu) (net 5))
 (segment (start 168.25 85.75) (end 168 86) (width 0.16) (layer B.Cu) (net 6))
 (segment (start 168 86) (end 168 87.8) (width 0.16) (layer B.Cu) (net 6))
 (segment (start 165.95 87.75) (end 164.7 87.75) (width 0.16) (layer B.Cu) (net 6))
 (segment (start 166.2 88) (end 165.95 87.75) (width 0.16) (layer B.Cu) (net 6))
 (segment (start 167.8 88) (end 166.2 88) (width 0.16) (layer B.Cu) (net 6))
 (segment (start 168 87.8) (end 167.8 88) (width 0.16) (layer B.Cu) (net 6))
 (via (at 159.5 85.75) (size 0.69) (drill 0.331) (layers F.Cu B.Cu) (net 6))
 (segment (start 159.87 82) (end 159.87 83.88) (width 0.16) (layer F.Cu) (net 6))
 (segment (start 159.75 84) (end 159.87 83.88) (width 0.16) (layer F.Cu) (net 6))
 (via (at 159.75 84) (size 0.69) (drill 0.331) (layers F.Cu B.Cu) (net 6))
 (segment (start 159.75 85.5) (end 159.75 84) (width 0.16) (layer B.Cu) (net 6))
 (segment (start 159.75 85.5) (end 159.5 85.75) (width 0.16) (layer B.Cu) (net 6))
 (segment (start 154.5 85.75) (end 152.25 85.75) (width 0.16) (layer F.Cu) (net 6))
 (segment (start 168.25 85.75) (end 159.5 85.75) (width 0.16) (layer F.Cu) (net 6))
 (segment (start 159.5 85.75) (end 154.5 85.75) (width 0.16) (layer F.Cu) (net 6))
 (via (at 168.25 85.75) (size 0.69) (drill 0.331) (layers F.Cu B.Cu) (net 6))
 (segment (start 151.12 84.62) (end 151.12 82) (width 0.16) (layer F.Cu) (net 6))
 (segment (start 152.25 85.75) (end 151.12 84.62) (width 0.16) (layer F.Cu) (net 6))
 (segment (start 168.62 83.88) (end 168.62 82) (width 0.16) (layer F.Cu) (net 6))
 (segment (start 168.5 84) (end 168.62 83.88) (width 0.16) (layer F.Cu) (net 6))
 (via (at 168.5 84) (size 0.69) (drill 0.331) (layers F.Cu B.Cu) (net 6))
 (segment (start 168.5 85.5) (end 168.5 84) (width 0.16) (layer B.Cu) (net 6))
 (segment (start 168.25 85.75) (end 168.5 85.5) (width 0.16) (layer B.Cu) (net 6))
 (segment (start 152.56 82) (end 152.56 83.81) (width 0.16) (layer F.Cu) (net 7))
 (via (at 154.25 86.75) (size 0.69) (drill 0.331) (layers F.Cu B.Cu) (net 7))
 (segment (start 152.75 85.25) (end 154.25 86.75) (width 0.16) (layer B.Cu) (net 7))
 (segment (start 152.75 84) (end 152.75 85.25) (width 0.16) (layer B.Cu) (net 7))
 (via (at 152.75 84) (size 0.69) (drill 0.331) (layers F.Cu B.Cu) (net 7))
 (segment (start 152.56 83.81) (end 152.75 84) (width 0.16) (layer F.Cu) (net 7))
 (via (at 165.75 86.75) (size 0.69) (drill 0.331) (layers F.Cu B.Cu) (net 7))
 (segment (start 165.75 86.75) (end 164.7 86.75) (width 0.16) (layer B.Cu) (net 7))
 (segment (start 170.06 82) (end 170.06 83.94) (width 0.16) (layer F.Cu) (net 7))
 (segment (start 156 86.75) (end 154.25 86.75) (width 0.16) (layer F.Cu) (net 7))
 (segment (start 157 86.75) (end 156 86.75) (width 0.16) (layer F.Cu) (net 7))
 (segment (start 168.75 86.75) (end 165.75 86.75) (width 0.16) (layer F.Cu) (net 7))
 (segment (start 165.75 86.75) (end 157 86.75) (width 0.16) (layer F.Cu) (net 7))
 (via (at 168.75 86.75) (size 0.69) (drill 0.331) (layers F.Cu B.Cu) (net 7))
 (segment (start 170 85.5) (end 168.75 86.75) (width 0.16) (layer B.Cu) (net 7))
 (segment (start 170 84) (end 170 85.5) (width 0.16) (layer B.Cu) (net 7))
 (via (at 170 84) (size 0.69) (drill 0.331) (layers F.Cu B.Cu) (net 7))
 (segment (start 170.06 83.94) (end 170 84) (width 0.16) (layer F.Cu) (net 7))
 (segment (start 161.31 82) (end 161.31 83.81) (width 0.16) (layer F.Cu) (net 7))
 (segment (start 165 86.45) (end 164.7 86.75) (width 0.16) (layer B.Cu) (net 7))
 (segment (start 165 83.75) (end 165 86.45) (width 0.16) (layer B.Cu) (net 7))
 (segment (start 164.5 83.25) (end 165 83.75) (width 0.16) (layer B.Cu) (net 7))
 (segment (start 162.25 83.25) (end 164.5 83.25) (width 0.16) (layer B.Cu) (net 7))
 (segment (start 161.5 84) (end 162.25 83.25) (width 0.16) (layer B.Cu) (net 7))
 (via (at 161.5 84) (size 0.69) (drill 0.331) (layers F.Cu B.Cu) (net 7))
 (segment (start 161.31 83.81) (end 161.5 84) (width 0.16) (layer F.Cu) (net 7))
 (segment (start 164.25 84.25) (end 164.75 84.75) (width 0.16) (layer F.Cu) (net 8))
 (segment (start 172.94 84.06) (end 172.94 82) (width 0.16) (layer F.Cu) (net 8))
 (segment (start 172.25 84.75) (end 172.94 84.06) (width 0.16) (layer F.Cu) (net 8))
 (segment (start 164.75 84.75) (end 172.25 84.75) (width 0.16) (layer F.Cu) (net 8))
 (segment (start 155.44 82) (end 155.44 84.19) (width 0.16) (layer F.Cu) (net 8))
 (segment (start 163.75 84.75) (end 164.25 84.25) (width 0.16) (layer F.Cu) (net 8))
 (segment (start 156 84.75) (end 163.75 84.75) (width 0.16) (layer F.Cu) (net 8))
 (segment (start 155.44 84.19) (end 156 84.75) (width 0.16) (layer F.Cu) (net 8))
 (segment (start 164.19 82) (end 164.19 84.19) (width 0.16) (layer F.Cu) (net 8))
 (segment (start 164 84.5) (end 164 86.05) (width 0.16) (layer B.Cu) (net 8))
 (segment (start 164.25 84.25) (end 164 84.5) (width 0.16) (layer B.Cu) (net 8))
 (via (at 164.25 84.25) (size 0.69) (drill 0.331) (layers F.Cu B.Cu) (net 8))
 (segment (start 164.19 84.19) (end 164.25 84.25) (width 0.16) (layer F.Cu) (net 8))
 (segment (start 167.4 87.4) (end 157.8 87.4) (width 0.16) (layer F.Cu) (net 9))
 (segment (start 156.88 84.08) (end 156.88 82) (width 0.16) (layer F.Cu) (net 9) (status 800000))
 (segment (start 156.9 84.1) (end 156.88 84.08) (width 0.16) (layer F.Cu) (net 9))
 (via (at 156.9 84.1) (size 0.69) (drill 0.331) (layers F.Cu B.Cu) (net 9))
 (segment (start 156.9 86.5) (end 156.9 84.1) (width 0.16) (layer B.Cu) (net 9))
 (segment (start 157.8 87.4) (end 156.9 86.5) (width 0.16) (layer B.Cu) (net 9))
 (via (at 157.8 87.4) (size 0.69) (drill 0.331) (layers F.Cu B.Cu) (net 9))
 (segment (start 174.38 82) (end 174.38 83.22) (width 0.16) (layer F.Cu) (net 9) (status C00000))
 (segment (start 174.38 83.22) (end 170.2 87.4) (width 0.16) (layer F.Cu) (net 9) (status 400000))
 (segment (start 170.2 87.4) (end 167.4 87.4) (width 0.16) (layer F.Cu) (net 9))
 (via (at 167.4 87.4) (size 0.69) (drill 0.331) (layers F.Cu B.Cu) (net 9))
 (segment (start 167.4 87.4) (end 167.35 87.35) (width 0.16) (layer B.Cu) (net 9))
 (segment (start 167.35 87.35) (end 166.35 87.35) (width 0.16) (layer B.Cu) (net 9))
 (segment (start 166.35 87.35) (end 166.4 87.4) (width 0.16) (layer B.Cu) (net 9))
 (segment (start 166.4 87.4) (end 166.4 87.3) (width 0.16) (layer B.Cu) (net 9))
 (segment (start 166.5 87.2) (end 166.4 87.3) (width 0.16) (layer B.Cu) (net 9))
 (segment (start 166.4 87.3) (end 166.3 87.4) (width 0.16) (layer B.Cu) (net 9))
 (segment (start 166.3 87.4) (end 165.5 87.4) (width 0.16) (layer B.Cu) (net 9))
 (segment (start 165.5 87.4) (end 165.35 87.25) (width 0.16) (layer B.Cu) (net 9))
 (segment (start 165.35 87.25) (end 164.7 87.25) (width 0.16) (layer B.Cu) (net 9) (status 800000))
 (segment (start 165.63 82) (end 165.63 83.73) (width 0.16) (layer F.Cu) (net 9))
 (segment (start 165.35 87.25) (end 164.7 87.25) (width 0.16) (layer B.Cu) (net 9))
 (segment (start 165.5 87.4) (end 165.35 87.25) (width 0.16) (layer B.Cu) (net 9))
 (segment (start 166.5 85) (end 166.5 87.2) (width 0.16) (layer B.Cu) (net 9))
 (segment (start 165.9 84) (end 166.5 85) (width 0.16) (layer B.Cu) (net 9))
 (via (at 165.9 84) (size 0.69) (drill 0.331) (layers F.Cu B.Cu) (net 9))
 (segment (start 165.63 83.73) (end 165.9 84) (width 0.16) (layer F.Cu) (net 9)))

